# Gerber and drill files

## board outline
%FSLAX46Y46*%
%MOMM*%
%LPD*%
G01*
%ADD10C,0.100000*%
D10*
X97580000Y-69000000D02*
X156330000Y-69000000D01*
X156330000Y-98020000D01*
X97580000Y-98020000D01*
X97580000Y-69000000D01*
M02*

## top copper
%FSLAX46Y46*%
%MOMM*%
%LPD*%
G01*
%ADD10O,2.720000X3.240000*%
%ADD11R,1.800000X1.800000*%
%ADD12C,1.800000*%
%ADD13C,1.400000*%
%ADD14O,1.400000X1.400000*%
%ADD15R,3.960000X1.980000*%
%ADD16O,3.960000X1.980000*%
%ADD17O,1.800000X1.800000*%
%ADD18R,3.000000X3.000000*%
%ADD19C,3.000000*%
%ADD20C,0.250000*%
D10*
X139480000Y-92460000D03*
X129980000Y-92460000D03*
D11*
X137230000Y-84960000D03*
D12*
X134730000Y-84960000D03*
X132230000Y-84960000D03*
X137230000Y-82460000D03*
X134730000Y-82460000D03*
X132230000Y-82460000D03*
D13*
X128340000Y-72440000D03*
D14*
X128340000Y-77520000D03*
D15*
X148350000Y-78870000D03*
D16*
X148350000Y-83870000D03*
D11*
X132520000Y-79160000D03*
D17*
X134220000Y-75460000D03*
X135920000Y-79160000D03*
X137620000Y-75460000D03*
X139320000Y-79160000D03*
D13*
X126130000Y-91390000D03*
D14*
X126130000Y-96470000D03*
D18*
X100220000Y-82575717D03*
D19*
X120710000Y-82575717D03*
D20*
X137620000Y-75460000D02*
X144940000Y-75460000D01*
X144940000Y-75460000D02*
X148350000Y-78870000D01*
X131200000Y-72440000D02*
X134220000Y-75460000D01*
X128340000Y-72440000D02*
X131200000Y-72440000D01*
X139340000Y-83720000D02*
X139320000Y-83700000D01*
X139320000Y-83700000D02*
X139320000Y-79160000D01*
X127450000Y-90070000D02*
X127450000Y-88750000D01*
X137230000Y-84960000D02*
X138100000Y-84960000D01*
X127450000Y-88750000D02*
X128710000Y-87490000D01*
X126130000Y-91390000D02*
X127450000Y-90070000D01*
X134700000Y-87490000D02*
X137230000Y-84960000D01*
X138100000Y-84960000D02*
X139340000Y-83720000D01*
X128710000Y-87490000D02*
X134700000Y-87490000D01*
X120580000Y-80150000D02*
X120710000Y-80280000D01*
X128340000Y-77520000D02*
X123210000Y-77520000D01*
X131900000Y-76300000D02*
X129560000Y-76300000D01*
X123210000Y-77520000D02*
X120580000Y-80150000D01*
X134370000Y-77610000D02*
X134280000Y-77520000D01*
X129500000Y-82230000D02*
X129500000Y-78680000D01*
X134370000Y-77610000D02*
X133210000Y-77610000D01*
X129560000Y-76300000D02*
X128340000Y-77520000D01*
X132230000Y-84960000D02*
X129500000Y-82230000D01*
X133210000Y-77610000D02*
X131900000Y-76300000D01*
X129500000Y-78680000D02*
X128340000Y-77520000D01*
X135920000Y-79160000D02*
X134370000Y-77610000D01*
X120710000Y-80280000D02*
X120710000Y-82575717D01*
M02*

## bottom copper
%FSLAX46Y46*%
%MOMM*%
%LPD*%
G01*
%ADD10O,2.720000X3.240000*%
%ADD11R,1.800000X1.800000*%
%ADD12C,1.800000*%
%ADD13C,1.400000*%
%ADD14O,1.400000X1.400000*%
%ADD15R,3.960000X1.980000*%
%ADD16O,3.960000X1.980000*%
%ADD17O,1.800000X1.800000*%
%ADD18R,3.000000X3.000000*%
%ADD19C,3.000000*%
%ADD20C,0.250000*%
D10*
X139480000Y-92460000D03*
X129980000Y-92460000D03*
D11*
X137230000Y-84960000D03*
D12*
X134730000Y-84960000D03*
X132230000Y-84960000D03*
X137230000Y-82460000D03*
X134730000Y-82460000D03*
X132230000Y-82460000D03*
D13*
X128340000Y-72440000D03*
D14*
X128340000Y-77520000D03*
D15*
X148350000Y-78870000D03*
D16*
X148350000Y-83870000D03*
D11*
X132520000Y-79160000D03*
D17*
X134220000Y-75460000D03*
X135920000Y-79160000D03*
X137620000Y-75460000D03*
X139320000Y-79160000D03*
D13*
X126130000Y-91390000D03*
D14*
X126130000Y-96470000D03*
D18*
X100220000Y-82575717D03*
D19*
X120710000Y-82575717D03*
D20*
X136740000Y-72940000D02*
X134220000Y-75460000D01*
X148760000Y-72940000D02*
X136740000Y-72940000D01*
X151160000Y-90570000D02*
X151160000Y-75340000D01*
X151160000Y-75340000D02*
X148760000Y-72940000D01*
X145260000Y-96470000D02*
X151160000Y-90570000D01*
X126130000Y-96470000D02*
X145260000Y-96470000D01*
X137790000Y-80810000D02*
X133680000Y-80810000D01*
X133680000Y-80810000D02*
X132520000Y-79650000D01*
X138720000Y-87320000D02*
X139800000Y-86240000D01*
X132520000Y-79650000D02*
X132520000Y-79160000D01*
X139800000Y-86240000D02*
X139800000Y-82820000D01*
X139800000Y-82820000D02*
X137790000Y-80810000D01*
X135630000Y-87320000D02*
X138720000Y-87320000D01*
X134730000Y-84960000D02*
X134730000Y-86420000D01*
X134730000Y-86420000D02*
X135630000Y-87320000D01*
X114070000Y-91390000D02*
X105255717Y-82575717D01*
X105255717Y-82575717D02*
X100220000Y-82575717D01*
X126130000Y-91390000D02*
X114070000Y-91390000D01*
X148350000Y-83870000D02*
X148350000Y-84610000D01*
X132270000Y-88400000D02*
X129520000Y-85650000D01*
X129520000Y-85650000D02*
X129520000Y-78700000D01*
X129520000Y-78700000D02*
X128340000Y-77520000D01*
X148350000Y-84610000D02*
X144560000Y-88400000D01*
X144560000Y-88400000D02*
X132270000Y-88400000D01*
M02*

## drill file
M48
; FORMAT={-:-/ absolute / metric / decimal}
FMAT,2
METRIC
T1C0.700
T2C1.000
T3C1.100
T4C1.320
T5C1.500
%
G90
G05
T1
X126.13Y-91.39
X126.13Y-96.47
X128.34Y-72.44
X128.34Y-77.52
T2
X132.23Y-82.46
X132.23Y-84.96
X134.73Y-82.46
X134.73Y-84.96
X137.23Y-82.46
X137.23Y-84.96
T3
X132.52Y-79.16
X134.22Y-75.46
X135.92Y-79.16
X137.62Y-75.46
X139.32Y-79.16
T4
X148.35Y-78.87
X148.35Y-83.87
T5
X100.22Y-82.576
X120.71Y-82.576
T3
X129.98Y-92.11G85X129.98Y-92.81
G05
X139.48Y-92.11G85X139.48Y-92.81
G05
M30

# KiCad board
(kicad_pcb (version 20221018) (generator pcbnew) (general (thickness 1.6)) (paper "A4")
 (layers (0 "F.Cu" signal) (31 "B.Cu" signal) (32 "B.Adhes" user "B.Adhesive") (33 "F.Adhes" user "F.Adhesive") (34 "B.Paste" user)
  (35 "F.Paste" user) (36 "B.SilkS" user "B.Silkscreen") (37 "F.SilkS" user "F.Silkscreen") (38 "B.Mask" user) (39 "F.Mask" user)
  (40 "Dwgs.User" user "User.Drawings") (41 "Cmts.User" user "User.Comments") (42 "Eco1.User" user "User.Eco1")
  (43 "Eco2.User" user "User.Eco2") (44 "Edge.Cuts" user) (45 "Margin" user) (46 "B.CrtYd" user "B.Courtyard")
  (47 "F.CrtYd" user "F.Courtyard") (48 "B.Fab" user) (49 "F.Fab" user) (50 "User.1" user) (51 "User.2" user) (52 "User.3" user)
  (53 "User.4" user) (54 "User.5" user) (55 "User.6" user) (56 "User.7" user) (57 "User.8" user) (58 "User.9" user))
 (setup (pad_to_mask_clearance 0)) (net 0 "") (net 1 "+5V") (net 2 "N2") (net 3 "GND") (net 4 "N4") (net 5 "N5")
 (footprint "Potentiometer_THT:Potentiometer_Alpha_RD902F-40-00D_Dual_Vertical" (layer "F.Cu") (at 137.23 84.96 -90)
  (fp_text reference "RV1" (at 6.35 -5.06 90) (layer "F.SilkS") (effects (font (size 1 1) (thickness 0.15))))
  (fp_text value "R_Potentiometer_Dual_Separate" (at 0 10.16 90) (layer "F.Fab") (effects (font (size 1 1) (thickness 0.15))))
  (pad "" thru_hole oval (at 7.5 -2.25) (size 2.72 3.24) (drill oval 1.1 1.8) (layers "*.Cu" "*.Mask"))
  (pad "" thru_hole oval (at 7.5 7.25) (size 2.72 3.24) (drill oval 1.1 1.8) (layers "*.Cu" "*.Mask"))
  (pad "1" thru_hole rect (at 0 0) (size 1.8 1.8) (drill 1) (layers "*.Cu" "*.Mask") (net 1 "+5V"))
  (pad "2" thru_hole circle (at 0 2.5) (size 1.8 1.8) (drill 1) (layers "*.Cu" "*.Mask") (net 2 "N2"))
  (pad "3" thru_hole circle (at 0 5) (size 1.8 1.8) (drill 1) (layers "*.Cu" "*.Mask") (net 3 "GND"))
  (pad "4" thru_hole circle (at -2.5 0) (size 1.8 1.8) (drill 1) (layers "*.Cu" "*.Mask"))
  (pad "5" thru_hole circle (at -2.5 2.5) (size 1.8 1.8) (drill 1) (layers "*.Cu" "*.Mask"))
  (pad "6" thru_hole circle (at -2.5 5) (size 1.8 1.8) (drill 1) (layers "*.Cu" "*.Mask")))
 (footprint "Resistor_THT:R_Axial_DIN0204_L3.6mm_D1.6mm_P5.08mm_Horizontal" (layer "F.Cu") (at 128.34 72.44 -90)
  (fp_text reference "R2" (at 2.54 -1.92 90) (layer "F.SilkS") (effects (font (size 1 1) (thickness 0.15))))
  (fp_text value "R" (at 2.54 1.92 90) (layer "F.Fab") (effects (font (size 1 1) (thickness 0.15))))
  (pad "1" thru_hole circle (at 0 0 270) (size 1.4 1.4) (drill 0.7) (layers "*.Cu" "*.Mask") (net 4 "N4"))
  (pad "2" thru_hole oval (at 5.08 0 270) (size 1.4 1.4) (drill 0.7) (layers "*.Cu" "*.Mask") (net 3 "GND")))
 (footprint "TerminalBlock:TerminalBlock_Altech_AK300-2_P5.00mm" (layer "F.Cu") (at 148.35 78.87 -90)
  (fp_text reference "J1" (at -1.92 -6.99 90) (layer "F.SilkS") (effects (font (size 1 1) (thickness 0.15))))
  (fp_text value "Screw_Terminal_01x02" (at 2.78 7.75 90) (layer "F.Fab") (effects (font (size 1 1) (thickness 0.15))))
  (pad "1" thru_hole rect (at 0 0 270) (size 1.98 3.96) (drill 1.32) (layers "*.Cu" "*.Mask") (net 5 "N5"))
  (pad "2" thru_hole oval (at 5 0 270) (size 1.98 3.96) (drill 1.32) (layers "*.Cu" "*.Mask") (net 3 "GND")))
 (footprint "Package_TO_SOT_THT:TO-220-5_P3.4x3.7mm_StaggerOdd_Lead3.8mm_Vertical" (layer "F.Cu") (at 132.52 79.16)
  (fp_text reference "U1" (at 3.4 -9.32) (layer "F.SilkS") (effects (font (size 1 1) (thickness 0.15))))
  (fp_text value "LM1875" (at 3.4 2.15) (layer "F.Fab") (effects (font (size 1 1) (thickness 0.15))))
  (pad "1" thru_hole rect (at 0 0) (size 1.8 1.8) (drill 1.1) (layers "*.Cu" "*.Mask") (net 2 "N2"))
  (pad "2" thru_hole oval (at 1.7 -3.7) (size 1.8 1.8) (drill 1.1) (layers "*.Cu" "*.Mask") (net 4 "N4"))
  (pad "3" thru_hole oval (at 3.4 0) (size 1.8 1.8) (drill 1.1) (layers "*.Cu" "*.Mask") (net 3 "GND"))
  (pad "4" thru_hole oval (at 5.1 -3.7) (size 1.8 1.8) (drill 1.1) (layers "*.Cu" "*.Mask") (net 5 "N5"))
  (pad "5" thru_hole oval (at 6.8 0) (size 1.8 1.8) (drill 1.1) (layers "*.Cu" "*.Mask") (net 1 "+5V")))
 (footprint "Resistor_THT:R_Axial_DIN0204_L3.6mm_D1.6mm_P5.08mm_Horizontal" (layer "F.Cu") (at 126.13 91.39 -90)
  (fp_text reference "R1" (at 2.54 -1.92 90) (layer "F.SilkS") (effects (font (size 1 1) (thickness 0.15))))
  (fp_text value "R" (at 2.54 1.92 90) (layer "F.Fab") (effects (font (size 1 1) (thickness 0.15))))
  (pad "1" thru_hole circle (at 0 0 270) (size 1.4 1.4) (drill 0.7) (layers "*.Cu" "*.Mask") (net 1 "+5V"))
  (pad "2" thru_hole oval (at 5.08 0 270) (size 1.4 1.4) (drill 0.7) (layers "*.Cu" "*.Mask") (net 4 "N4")))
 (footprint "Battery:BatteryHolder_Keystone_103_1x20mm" (layer "F.Cu") (at 100.22 82.575717)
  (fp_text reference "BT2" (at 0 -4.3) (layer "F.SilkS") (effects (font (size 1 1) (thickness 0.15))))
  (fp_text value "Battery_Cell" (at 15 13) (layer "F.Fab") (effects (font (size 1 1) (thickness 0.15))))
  (pad "1" thru_hole rect (at 0 0) (size 3 3) (drill 1.5) (layers "*.Cu" "*.Mask") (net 1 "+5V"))
  (pad "2" thru_hole circle (at 20.49 0) (size 3 3) (drill 1.5) (layers "*.Cu" "*.Mask") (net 3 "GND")))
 (gr_rect (start 97.58 69) (end 156.33 98.02) (stroke (width 0.1) (type default)) (fill none) (layer "Edge.Cuts"))
 (segment (start 137.62 75.46) (end 144.94 75.46) (width 0.25) (layer "F.Cu") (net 5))
 (segment (start 144.94 75.46) (end 148.35 78.87) (width 0.25) (layer "F.Cu") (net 5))
 (segment (start 131.2 72.44) (end 134.22 75.46) (width 0.25) (layer "F.Cu") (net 4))
 (segment (start 128.34 72.44) (end 131.2 72.44) (width 0.25) (layer "F.Cu") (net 4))
 (segment (start 136.74 72.94) (end 134.22 75.46) (width 0.25) (layer "B.Cu") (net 4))
 (segment (start 148.76 72.94) (end 136.74 72.94) (width 0.25) (layer "B.Cu") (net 4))
 (segment (start 151.16 90.57) (end 151.16 75.34) (width 0.25) (layer "B.Cu") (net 4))
 (segment (start 151.16 75.34) (end 148.76 72.94) (width 0.25) (layer "B.Cu") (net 4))
 (segment (start 145.26 96.47) (end 151.16 90.57) (width 0.25) (layer "B.Cu") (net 4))
 (segment (start 126.13 96.47) (end 145.26 96.47) (width 0.25) (layer "B.Cu") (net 4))
 (segment (start 137.79 80.81) (end 133.68 80.81) (width 0.25) (layer "B.Cu") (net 2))
 (segment (start 133.68 80.81) (end 132.52 79.65) (width 0.25) (layer "B.Cu") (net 2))
 (segment (start 138.72 87.32) (end 139.8 86.24) (width 0.25) (layer "B.Cu") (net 2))
 (segment (start 132.52 79.65) (end 132.52 79.16) (width 0.25) (layer "B.Cu") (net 2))
 (segment (start 139.8 86.24) (end 139.8 82.82) (width 0.25) (layer "B.Cu") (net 2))
 (segment (start 139.8 82.82) (end 137.79 80.81) (width 0.25) (layer "B.Cu") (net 2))
 (segment (start 135.63 87.32) (end 138.72 87.32) (width 0.25) (layer "B.Cu") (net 2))
 (segment (start 134.73 84.96) (end 134.73 86.42) (width 0.25) (layer "B.Cu") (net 2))
 (segment (start 134.73 86.42) (end 135.63 87.32) (width 0.25) (layer "B.Cu") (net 2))
 (segment (start 139.34 83.72) (end 139.32 83.7) (width 0.25) (layer "F.Cu") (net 1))
 (segment (start 139.32 83.7) (end 139.32 79.16) (width 0.25) (layer "F.Cu") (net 1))
 (segment (start 127.45 90.07) (end 127.45 88.75) (width 0.25) (layer "F.Cu") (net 1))
 (segment (start 137.23 84.96) (end 138.1 84.96) (width 0.25) (layer "F.Cu") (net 1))
 (segment (start 127.45 88.75) (end 128.71 87.49) (width 0.25) (layer "F.Cu") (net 1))
 (segment (start 126.13 91.39) (end 127.45 90.07) (width 0.25) (layer "F.Cu") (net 1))
 (segment (start 134.7 87.49) (end 137.23 84.96) (width 0.25) (layer "F.Cu") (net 1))
 (segment (start 138.1 84.96) (end 139.34 83.72) (width 0.25) (layer "F.Cu") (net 1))
 (segment (start 128.71 87.49) (end 134.7 87.49) (width 0.25) (layer "F.Cu") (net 1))
 (segment (start 114.07 91.39) (end 105.255717 82.575717) (width 0.25) (layer "B.Cu") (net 1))
 (segment (start 105.255717 82.575717) (end 100.22 82.575717) (width 0.25) (layer "B.Cu") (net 1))
 (segment (start 126.13 91.39) (end 114.07 91.39) (width 0.25) (layer "B.Cu") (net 1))
 (segment (start 120.58 80.15) (end 120.71 80.28) (width 0.25) (layer "F.Cu") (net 3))
 (segment (start 128.34 77.52) (end 123.21 77.52) (width 0.25) (layer "F.Cu") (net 3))
 (segment (start 131.9 76.3) (end 129.56 76.3) (width 0.25) (layer "F.Cu") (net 3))
 (segment (start 123.21 77.52) (end 120.58 80.15) (width 0.25) (layer "F.Cu") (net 3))
 (segment (start 134.37 77.61) (end 134.28 77.52) (width 0.25) (layer "F.Cu") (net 3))
 (segment (start 129.5 82.23) (end 129.5 78.68) (width 0.25) (layer "F.Cu") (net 3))
 (segment (start 134.37 77.61) (end 133.21 77.61) (width 0.25) (layer "F.Cu") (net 3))
 (segment (start 129.56 76.3) (end 128.34 77.52) (width 0.25) (layer "F.Cu") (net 3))
 (segment (start 132.23 84.96) (end 129.5 82.23) (width 0.25) (layer "F.Cu") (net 3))
 (segment (start 133.21 77.61) (end 131.9 76.3) (width 0.25) (layer "F.Cu") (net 3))
 (segment (start 129.5 78.68) (end 128.34 77.52) (width 0.25) (layer "F.Cu") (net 3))
 (segment (start 135.92 79.16) (end 134.37 77.61) (width 0.25) (layer "F.Cu") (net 3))
 (segment (start 120.71 80.28) (end 120.71 82.575717) (width 0.25) (layer "F.Cu") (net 3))
 (segment (start 148.35 83.87) (end 148.35 84.61) (width 0.25) (layer "B.Cu") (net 3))
 (segment (start 132.27 88.4) (end 129.52 85.65) (width 0.25) (layer "B.Cu") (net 3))
 (segment (start 129.52 85.65) (end 129.52 78.7) (width 0.25) (layer "B.Cu") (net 3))
 (segment (start 129.52 78.7) (end 128.34 77.52) (width 0.25) (layer "B.Cu") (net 3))
 (segment (start 148.35 84.61) (end 144.56 88.4) (width 0.25) (layer "B.Cu") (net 3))
 (segment (start 144.56 88.4) (end 132.27 88.4) (width 0.25) (layer "B.Cu") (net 3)))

